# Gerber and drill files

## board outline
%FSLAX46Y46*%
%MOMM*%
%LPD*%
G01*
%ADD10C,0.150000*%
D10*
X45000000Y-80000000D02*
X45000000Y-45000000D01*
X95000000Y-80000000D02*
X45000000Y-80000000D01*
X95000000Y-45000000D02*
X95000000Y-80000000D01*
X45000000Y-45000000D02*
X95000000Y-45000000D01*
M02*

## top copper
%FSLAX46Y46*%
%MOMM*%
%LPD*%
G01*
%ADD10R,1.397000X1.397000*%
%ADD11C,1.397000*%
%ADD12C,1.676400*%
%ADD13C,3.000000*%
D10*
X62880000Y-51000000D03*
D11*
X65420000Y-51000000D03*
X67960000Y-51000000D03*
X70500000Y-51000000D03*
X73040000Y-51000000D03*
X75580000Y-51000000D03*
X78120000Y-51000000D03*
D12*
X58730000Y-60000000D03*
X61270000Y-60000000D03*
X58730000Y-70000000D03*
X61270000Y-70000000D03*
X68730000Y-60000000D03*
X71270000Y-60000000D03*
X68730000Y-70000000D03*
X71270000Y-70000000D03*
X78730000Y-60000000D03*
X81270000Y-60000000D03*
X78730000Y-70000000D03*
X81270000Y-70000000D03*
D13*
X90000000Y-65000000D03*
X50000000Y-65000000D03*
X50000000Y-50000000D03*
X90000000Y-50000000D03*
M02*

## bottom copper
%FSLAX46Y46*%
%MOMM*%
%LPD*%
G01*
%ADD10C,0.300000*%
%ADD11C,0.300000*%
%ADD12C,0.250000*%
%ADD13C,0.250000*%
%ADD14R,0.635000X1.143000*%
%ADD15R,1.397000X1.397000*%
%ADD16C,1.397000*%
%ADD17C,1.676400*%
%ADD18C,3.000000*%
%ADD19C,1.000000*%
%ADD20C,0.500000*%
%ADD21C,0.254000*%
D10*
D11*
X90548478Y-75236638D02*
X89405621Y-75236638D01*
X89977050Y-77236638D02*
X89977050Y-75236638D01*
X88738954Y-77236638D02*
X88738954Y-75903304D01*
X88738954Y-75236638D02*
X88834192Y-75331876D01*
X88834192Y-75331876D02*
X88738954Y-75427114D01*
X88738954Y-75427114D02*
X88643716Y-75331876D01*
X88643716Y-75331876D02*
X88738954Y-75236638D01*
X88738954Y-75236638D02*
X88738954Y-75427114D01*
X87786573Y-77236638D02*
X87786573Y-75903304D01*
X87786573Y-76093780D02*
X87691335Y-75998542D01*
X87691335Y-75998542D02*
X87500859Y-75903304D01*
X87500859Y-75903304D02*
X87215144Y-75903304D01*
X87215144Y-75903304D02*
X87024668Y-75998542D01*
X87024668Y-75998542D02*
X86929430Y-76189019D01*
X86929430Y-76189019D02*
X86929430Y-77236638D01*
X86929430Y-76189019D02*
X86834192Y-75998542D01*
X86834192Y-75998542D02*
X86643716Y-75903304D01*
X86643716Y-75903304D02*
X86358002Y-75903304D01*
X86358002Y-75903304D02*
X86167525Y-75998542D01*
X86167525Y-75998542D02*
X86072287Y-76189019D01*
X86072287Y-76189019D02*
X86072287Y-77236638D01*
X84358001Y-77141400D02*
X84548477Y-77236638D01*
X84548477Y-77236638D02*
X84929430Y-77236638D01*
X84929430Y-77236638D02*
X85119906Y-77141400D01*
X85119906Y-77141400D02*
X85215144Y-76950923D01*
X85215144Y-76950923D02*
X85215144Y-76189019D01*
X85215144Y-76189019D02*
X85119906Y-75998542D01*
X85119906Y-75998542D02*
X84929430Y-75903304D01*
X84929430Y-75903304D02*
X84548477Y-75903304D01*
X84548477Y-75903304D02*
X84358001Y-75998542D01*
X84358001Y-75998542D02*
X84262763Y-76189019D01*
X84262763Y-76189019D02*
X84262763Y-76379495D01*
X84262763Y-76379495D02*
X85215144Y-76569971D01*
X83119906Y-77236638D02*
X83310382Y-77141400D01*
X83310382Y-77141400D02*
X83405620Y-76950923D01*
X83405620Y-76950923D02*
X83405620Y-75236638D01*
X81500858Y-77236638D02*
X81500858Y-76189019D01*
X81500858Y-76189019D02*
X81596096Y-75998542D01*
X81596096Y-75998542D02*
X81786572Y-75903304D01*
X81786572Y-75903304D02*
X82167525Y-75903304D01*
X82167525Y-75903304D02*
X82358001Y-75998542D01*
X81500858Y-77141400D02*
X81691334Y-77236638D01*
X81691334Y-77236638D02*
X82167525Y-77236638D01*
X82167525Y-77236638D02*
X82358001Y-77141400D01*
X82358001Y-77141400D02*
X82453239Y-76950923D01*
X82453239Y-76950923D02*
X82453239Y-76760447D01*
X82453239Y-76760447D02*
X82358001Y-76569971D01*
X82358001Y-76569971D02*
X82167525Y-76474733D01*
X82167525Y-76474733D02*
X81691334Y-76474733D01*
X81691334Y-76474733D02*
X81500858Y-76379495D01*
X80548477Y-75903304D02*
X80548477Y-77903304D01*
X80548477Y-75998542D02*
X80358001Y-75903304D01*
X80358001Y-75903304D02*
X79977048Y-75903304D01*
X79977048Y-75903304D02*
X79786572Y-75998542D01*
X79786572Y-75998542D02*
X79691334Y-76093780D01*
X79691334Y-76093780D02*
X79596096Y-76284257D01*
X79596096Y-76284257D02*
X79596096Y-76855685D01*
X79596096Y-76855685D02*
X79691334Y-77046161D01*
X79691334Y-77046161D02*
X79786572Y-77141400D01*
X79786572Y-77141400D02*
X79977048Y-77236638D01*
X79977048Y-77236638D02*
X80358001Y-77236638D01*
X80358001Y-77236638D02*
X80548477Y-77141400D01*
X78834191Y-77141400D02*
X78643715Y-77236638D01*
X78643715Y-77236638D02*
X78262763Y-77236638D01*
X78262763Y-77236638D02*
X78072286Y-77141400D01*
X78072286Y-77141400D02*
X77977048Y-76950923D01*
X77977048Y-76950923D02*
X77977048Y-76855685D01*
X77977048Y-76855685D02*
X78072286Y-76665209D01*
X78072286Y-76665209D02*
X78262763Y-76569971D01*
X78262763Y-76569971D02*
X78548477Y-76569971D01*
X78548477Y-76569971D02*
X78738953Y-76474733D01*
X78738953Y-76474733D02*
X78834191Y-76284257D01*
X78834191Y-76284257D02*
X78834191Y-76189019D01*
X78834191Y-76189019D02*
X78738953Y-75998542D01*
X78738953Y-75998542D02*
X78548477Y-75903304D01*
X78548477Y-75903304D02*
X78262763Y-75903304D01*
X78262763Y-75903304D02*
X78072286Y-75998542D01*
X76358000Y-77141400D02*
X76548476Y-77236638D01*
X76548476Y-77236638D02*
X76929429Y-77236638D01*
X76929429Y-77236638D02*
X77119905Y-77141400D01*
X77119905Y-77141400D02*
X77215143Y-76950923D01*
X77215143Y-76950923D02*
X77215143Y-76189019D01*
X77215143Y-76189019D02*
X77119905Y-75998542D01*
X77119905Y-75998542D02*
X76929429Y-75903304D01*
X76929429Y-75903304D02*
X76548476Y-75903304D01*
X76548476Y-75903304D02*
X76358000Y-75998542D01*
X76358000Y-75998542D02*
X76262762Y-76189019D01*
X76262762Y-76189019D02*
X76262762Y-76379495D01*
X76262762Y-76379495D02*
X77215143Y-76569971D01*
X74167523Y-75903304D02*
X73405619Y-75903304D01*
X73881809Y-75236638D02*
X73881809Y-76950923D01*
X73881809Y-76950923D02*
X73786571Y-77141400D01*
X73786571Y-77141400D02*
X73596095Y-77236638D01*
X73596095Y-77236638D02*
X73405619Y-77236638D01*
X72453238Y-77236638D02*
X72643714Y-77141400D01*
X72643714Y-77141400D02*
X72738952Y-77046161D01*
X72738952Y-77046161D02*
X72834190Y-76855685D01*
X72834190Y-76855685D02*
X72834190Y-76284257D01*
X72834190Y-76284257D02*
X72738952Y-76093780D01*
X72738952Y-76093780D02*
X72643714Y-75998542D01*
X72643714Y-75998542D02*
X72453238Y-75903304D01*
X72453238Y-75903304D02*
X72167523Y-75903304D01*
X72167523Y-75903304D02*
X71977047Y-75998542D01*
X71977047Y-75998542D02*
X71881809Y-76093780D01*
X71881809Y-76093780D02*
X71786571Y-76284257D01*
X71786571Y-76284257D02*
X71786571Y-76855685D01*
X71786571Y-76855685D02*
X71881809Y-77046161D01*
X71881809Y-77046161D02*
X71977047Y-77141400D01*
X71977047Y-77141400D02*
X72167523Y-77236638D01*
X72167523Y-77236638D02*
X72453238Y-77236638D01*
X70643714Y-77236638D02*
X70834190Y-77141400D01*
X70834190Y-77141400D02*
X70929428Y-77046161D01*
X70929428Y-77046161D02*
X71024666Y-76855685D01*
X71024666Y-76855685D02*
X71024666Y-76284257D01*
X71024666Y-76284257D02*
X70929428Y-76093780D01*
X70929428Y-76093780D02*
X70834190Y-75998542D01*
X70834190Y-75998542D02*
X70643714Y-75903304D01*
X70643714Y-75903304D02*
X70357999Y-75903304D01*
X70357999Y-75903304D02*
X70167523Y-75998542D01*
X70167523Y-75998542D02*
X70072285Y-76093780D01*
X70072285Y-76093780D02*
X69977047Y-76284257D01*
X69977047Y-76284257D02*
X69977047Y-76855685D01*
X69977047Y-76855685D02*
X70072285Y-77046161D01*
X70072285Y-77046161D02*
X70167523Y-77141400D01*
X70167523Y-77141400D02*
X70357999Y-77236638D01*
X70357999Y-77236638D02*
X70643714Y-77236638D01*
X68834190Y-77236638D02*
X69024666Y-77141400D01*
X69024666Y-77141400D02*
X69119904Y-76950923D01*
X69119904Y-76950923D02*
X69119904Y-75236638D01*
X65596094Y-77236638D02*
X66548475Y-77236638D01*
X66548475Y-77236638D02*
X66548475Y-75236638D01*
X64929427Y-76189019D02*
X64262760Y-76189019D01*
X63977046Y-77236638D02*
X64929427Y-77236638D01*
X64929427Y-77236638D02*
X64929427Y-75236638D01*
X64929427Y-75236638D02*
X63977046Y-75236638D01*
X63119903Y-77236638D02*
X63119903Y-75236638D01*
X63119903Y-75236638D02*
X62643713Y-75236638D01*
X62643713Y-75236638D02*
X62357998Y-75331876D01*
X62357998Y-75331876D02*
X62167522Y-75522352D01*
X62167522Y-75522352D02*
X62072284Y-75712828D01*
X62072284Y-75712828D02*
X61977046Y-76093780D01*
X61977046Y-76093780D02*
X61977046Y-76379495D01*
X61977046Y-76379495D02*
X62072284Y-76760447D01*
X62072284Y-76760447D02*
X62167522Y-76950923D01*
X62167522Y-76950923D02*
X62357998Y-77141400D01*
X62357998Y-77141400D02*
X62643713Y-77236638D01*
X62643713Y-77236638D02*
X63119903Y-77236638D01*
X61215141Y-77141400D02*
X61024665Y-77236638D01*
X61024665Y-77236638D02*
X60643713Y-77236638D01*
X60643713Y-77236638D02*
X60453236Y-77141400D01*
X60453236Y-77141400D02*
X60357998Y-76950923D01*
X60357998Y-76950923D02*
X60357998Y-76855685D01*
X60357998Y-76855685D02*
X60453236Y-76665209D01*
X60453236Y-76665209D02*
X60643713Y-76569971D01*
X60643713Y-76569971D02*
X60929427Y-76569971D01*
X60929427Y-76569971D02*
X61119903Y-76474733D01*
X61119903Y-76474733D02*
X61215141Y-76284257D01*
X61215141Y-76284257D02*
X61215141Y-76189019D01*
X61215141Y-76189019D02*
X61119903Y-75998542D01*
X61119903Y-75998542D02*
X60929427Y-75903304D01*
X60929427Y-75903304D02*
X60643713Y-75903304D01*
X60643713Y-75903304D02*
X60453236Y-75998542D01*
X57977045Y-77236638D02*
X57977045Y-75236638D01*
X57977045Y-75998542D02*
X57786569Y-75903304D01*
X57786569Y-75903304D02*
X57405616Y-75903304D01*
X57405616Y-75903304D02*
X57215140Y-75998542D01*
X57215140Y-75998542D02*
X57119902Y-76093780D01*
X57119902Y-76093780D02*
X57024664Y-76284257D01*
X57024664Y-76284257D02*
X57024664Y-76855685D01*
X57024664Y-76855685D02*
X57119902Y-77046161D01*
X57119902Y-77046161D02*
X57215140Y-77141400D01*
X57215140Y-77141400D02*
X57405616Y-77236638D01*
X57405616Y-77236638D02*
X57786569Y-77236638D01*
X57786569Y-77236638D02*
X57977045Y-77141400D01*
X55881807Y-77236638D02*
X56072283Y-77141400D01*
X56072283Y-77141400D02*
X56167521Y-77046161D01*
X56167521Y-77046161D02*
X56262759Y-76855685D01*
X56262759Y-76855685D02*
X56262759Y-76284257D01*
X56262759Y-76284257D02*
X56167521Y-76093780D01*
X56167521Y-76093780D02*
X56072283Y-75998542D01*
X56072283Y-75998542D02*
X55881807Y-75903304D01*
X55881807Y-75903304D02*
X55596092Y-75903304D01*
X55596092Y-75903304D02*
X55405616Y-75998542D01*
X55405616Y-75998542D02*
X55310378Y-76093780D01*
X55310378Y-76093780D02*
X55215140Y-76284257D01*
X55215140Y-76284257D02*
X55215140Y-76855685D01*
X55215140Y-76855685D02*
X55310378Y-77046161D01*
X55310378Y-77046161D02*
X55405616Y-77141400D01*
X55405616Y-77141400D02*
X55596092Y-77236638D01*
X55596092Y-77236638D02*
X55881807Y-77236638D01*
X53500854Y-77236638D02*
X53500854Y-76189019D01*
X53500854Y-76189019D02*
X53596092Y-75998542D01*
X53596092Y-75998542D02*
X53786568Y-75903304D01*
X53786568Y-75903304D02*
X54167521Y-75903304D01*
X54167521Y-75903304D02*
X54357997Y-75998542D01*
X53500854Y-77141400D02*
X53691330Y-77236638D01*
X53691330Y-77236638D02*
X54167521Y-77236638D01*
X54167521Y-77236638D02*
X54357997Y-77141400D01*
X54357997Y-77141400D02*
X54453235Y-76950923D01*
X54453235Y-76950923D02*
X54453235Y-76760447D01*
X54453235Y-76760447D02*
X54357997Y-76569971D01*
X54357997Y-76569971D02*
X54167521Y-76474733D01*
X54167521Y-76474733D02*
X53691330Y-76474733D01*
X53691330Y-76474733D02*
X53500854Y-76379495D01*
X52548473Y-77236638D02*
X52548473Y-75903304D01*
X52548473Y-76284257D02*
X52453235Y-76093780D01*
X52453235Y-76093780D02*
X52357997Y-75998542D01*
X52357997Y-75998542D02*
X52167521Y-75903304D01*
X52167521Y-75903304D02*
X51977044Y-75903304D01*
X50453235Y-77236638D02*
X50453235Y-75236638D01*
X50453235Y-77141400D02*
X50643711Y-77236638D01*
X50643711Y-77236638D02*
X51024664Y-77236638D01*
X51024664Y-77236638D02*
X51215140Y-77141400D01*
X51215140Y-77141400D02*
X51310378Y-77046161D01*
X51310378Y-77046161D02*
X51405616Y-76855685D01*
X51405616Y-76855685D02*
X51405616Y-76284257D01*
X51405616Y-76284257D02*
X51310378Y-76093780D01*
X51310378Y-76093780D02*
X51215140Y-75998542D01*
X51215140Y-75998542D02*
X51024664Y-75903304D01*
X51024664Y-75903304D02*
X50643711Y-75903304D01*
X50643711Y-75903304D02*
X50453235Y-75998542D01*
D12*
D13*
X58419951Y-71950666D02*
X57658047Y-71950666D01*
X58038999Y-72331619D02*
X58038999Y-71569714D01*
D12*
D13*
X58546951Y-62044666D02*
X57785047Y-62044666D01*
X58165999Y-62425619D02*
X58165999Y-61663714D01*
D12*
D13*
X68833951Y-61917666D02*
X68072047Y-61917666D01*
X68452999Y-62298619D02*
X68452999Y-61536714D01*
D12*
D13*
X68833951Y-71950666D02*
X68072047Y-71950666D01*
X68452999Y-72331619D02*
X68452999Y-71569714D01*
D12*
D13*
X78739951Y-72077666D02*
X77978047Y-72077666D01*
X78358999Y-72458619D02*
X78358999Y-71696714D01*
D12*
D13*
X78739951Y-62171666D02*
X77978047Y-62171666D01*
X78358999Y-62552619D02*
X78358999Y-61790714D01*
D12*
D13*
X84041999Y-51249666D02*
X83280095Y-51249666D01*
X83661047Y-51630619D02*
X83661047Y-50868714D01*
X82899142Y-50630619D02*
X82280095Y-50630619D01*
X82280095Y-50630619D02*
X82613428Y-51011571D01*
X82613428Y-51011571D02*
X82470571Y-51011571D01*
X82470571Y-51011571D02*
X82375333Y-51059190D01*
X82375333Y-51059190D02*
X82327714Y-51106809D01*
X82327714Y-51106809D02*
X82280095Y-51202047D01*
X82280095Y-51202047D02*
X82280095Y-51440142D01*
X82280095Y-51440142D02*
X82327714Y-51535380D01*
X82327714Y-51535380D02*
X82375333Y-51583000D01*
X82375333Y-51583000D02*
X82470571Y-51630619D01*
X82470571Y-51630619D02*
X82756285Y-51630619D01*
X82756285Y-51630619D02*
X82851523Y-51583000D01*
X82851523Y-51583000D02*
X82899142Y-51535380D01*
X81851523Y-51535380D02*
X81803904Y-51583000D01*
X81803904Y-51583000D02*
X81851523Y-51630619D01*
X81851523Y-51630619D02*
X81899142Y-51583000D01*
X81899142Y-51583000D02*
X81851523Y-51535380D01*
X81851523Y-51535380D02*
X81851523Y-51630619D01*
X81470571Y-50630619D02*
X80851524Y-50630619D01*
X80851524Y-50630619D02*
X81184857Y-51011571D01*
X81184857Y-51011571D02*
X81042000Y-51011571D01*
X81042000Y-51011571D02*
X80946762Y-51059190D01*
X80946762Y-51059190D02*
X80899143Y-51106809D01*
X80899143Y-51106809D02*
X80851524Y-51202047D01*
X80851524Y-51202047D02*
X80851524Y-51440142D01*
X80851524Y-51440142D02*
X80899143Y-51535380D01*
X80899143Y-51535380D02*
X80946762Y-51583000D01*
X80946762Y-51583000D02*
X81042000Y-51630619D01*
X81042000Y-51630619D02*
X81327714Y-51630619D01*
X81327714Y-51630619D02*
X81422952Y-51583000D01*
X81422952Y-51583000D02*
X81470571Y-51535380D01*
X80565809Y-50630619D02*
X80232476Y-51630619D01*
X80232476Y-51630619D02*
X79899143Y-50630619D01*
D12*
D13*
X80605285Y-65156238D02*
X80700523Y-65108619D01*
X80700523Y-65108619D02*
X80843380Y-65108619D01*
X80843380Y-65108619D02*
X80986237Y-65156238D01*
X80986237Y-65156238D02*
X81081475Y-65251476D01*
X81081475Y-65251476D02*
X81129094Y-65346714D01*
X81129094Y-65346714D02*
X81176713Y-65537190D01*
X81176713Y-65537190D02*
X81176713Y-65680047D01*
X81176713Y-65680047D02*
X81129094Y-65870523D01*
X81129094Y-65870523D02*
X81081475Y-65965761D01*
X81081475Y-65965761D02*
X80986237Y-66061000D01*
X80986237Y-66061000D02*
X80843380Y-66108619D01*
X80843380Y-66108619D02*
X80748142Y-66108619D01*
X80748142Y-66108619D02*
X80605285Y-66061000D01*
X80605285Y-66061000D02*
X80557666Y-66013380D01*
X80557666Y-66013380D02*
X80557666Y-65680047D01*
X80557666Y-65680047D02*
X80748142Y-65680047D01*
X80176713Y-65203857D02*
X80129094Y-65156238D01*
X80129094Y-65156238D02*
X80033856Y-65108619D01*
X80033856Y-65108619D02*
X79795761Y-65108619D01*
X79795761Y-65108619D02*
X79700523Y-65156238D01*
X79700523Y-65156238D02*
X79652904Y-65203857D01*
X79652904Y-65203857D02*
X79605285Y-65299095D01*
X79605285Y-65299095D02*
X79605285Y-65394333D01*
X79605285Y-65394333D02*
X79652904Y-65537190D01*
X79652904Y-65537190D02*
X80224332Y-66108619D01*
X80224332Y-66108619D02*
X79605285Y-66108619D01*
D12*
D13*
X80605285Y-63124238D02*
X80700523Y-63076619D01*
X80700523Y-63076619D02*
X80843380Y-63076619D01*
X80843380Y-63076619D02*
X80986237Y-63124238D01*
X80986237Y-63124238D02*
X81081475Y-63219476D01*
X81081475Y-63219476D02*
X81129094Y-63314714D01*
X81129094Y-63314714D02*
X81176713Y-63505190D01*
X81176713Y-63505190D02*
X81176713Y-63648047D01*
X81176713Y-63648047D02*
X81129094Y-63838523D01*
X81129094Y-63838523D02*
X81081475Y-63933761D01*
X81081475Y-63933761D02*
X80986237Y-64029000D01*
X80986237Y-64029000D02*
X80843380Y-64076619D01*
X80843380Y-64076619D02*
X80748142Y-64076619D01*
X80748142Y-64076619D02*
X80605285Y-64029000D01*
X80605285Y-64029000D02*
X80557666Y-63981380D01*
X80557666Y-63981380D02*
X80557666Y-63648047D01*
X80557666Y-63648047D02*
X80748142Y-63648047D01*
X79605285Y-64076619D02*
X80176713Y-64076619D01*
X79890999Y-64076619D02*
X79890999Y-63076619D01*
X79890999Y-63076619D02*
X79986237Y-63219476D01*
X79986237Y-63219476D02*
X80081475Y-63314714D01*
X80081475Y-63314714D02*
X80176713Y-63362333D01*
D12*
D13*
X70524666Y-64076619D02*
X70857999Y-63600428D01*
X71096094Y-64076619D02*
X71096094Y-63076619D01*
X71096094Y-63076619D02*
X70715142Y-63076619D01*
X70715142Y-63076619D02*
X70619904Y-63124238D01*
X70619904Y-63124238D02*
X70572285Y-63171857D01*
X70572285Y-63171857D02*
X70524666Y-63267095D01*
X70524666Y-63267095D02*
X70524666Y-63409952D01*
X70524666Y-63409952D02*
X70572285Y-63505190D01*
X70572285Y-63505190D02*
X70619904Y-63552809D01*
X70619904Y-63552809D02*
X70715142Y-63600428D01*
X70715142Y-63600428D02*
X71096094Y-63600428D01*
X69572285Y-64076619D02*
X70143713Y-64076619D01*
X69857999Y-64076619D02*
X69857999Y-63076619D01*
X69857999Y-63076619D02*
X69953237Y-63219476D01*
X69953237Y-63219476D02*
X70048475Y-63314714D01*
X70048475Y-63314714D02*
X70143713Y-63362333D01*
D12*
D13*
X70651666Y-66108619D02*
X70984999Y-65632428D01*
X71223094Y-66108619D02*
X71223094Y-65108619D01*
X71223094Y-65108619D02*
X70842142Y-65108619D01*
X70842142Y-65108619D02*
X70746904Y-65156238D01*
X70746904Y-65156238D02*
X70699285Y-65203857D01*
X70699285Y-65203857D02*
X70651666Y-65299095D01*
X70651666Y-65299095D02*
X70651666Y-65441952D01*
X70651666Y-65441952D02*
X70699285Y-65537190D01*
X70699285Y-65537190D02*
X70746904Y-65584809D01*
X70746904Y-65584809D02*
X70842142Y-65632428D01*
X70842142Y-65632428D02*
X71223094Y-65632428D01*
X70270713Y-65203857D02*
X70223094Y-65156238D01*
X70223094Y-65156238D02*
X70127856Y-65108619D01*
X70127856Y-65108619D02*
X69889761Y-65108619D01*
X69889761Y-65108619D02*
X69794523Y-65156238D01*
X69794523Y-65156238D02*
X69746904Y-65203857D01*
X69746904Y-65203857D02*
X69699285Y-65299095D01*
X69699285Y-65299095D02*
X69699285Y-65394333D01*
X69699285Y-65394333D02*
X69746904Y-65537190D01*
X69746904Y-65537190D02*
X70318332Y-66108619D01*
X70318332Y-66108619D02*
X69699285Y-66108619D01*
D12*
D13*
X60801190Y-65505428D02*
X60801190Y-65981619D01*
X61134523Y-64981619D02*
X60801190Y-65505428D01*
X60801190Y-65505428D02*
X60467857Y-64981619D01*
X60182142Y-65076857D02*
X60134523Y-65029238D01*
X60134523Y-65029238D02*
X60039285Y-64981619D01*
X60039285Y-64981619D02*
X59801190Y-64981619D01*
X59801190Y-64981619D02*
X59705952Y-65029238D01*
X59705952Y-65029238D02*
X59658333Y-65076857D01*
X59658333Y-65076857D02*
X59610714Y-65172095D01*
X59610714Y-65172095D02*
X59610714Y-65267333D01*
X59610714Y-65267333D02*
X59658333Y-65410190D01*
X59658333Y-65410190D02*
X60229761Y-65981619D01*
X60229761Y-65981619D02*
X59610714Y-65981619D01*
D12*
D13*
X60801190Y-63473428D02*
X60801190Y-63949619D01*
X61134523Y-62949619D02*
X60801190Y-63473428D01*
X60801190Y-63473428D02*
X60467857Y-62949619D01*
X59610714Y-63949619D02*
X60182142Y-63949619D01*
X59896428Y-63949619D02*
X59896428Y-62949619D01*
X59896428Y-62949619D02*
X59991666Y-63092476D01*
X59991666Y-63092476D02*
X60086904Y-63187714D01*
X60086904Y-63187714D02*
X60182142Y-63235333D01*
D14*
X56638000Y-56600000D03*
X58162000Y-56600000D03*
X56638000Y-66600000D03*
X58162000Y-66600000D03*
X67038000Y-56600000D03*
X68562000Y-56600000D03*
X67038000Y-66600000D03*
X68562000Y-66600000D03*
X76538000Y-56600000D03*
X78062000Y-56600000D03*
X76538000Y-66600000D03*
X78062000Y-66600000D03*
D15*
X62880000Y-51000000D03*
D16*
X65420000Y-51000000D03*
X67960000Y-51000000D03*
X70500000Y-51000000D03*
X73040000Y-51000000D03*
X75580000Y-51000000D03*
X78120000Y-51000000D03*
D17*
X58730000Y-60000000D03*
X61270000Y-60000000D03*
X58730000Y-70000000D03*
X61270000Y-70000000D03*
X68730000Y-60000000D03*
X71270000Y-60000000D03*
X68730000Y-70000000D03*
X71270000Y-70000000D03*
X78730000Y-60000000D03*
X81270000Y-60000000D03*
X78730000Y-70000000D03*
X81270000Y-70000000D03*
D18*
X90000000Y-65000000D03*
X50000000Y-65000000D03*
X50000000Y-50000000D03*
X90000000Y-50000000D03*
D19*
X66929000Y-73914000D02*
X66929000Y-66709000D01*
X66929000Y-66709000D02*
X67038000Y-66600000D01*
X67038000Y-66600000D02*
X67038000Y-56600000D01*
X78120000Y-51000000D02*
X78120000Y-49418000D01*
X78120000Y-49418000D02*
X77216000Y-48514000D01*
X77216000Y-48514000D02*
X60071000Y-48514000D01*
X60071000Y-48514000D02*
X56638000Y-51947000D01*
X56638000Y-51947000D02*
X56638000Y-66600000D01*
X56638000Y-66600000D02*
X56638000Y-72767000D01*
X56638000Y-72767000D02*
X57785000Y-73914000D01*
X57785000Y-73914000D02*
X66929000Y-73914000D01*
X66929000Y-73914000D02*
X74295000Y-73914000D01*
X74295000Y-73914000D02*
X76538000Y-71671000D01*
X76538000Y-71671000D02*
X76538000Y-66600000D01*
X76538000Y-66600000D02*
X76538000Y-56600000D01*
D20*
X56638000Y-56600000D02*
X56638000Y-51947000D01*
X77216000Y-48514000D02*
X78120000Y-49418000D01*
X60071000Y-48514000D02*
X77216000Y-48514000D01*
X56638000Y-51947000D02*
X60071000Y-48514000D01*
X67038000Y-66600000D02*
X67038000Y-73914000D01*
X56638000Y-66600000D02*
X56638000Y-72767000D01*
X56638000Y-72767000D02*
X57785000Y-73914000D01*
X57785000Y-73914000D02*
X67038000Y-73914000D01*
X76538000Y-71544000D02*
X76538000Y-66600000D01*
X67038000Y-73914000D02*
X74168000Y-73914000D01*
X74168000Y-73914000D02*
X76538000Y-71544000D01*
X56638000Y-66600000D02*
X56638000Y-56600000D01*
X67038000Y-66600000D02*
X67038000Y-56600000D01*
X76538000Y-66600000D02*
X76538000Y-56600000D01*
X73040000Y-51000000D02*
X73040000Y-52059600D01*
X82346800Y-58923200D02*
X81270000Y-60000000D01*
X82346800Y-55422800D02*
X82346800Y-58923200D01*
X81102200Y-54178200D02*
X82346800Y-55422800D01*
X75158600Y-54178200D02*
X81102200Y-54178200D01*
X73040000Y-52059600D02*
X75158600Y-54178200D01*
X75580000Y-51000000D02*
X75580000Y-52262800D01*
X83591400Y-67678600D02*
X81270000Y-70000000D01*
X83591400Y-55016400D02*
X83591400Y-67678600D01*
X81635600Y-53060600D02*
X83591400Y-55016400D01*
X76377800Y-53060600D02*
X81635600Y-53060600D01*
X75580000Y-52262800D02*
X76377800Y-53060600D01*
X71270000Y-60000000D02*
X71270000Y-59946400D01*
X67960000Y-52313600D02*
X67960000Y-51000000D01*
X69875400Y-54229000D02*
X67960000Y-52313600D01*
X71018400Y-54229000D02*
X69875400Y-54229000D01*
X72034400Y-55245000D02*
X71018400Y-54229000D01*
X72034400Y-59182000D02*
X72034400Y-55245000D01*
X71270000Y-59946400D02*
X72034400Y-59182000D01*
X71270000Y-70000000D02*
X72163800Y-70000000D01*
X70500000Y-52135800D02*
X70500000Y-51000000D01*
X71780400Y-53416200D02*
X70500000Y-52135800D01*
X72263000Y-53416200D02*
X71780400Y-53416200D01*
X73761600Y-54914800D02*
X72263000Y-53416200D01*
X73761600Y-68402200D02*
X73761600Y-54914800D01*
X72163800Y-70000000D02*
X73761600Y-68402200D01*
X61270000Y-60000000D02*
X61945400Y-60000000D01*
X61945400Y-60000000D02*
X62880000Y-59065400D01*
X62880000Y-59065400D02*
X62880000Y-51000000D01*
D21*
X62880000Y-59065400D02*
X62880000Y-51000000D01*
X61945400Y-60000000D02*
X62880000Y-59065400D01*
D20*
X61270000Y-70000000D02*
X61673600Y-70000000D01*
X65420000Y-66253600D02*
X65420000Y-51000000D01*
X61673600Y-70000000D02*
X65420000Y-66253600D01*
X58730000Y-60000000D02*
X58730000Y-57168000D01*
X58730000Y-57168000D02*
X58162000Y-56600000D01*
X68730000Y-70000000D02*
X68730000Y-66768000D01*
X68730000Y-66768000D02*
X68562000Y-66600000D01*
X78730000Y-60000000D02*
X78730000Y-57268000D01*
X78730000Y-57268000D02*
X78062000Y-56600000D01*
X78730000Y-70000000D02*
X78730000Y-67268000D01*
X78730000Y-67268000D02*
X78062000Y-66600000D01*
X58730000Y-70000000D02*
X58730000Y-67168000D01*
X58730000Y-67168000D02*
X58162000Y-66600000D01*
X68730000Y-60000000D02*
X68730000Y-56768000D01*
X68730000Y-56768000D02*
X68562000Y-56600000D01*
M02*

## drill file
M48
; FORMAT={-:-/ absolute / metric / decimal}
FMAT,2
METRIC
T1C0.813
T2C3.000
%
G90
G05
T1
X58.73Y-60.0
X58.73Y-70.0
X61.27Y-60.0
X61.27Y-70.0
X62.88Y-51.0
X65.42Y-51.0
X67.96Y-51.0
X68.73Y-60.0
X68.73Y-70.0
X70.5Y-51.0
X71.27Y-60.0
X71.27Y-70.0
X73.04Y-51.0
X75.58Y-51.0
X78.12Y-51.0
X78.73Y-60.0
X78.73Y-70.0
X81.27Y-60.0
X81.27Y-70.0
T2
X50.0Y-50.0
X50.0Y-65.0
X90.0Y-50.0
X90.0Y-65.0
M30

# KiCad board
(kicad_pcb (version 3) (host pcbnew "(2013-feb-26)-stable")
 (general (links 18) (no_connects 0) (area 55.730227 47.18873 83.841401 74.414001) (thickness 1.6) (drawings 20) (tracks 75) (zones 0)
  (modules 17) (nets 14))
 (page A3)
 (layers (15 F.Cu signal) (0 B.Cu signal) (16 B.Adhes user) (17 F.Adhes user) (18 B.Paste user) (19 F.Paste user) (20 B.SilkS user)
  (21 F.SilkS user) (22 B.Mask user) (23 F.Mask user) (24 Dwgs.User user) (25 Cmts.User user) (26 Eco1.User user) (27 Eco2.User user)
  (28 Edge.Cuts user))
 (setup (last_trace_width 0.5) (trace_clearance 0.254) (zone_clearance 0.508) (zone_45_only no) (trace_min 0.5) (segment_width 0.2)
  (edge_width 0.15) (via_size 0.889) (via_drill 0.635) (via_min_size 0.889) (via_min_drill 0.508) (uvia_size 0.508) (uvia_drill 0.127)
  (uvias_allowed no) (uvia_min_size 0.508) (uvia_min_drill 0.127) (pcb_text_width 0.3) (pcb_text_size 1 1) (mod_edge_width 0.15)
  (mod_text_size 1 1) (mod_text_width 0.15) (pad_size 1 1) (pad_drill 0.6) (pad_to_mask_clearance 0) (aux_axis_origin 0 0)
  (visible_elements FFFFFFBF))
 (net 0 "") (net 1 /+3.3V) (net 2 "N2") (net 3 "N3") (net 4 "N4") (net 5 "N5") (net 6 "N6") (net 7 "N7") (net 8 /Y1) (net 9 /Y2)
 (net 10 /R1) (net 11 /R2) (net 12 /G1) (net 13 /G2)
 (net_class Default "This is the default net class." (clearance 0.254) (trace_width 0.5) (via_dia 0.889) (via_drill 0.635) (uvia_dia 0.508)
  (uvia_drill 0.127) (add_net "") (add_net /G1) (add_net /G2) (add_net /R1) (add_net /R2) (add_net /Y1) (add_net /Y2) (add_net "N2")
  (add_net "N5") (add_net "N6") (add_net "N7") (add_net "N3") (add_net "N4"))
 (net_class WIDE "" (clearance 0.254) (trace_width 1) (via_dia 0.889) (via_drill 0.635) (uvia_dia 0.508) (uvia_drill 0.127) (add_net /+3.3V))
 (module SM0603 (layer B.Cu) (at 57.4 56.6)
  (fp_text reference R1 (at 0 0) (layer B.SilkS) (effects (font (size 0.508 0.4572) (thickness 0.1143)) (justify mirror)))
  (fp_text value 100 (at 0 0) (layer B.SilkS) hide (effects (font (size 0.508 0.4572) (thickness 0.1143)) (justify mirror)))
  (pad 1 smd rect (at -0.762 0) (size 0.635 1.143) (layers B.Cu B.Paste B.Mask) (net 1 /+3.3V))
  (pad 2 smd rect (at 0.762 0) (size 0.635 1.143) (layers B.Cu B.Paste B.Mask) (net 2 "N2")))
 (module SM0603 (layer B.Cu) (at 57.4 66.6)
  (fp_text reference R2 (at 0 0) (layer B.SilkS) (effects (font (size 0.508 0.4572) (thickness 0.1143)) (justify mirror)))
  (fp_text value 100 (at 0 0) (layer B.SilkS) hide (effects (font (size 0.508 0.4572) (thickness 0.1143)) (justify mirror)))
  (pad 1 smd rect (at -0.762 0) (size 0.635 1.143) (layers B.Cu B.Paste B.Mask) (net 1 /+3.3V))
  (pad 2 smd rect (at 0.762 0) (size 0.635 1.143) (layers B.Cu B.Paste B.Mask) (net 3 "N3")))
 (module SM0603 (layer B.Cu) (at 67.8 56.6)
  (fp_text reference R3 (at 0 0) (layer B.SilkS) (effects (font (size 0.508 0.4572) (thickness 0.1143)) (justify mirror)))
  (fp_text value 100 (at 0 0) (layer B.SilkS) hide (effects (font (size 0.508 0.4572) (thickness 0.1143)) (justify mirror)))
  (pad 1 smd rect (at -0.762 0) (size 0.635 1.143) (layers B.Cu B.Paste B.Mask) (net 1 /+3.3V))
  (pad 2 smd rect (at 0.762 0) (size 0.635 1.143) (layers B.Cu B.Paste B.Mask) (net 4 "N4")))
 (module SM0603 (layer B.Cu) (at 67.8 66.6)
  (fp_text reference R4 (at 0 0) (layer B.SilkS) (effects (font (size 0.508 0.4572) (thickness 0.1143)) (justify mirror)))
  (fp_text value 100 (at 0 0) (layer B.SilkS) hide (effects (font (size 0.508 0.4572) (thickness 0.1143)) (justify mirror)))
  (pad 1 smd rect (at -0.762 0) (size 0.635 1.143) (layers B.Cu B.Paste B.Mask) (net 1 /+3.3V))
  (pad 2 smd rect (at 0.762 0) (size 0.635 1.143) (layers B.Cu B.Paste B.Mask) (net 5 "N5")))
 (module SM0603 (layer B.Cu) (at 77.3 56.6)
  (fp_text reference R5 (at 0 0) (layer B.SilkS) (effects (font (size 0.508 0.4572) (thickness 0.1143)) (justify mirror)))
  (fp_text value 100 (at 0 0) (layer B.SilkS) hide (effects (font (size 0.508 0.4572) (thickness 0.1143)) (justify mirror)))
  (pad 1 smd rect (at -0.762 0) (size 0.635 1.143) (layers B.Cu B.Paste B.Mask) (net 1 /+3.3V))
  (pad 2 smd rect (at 0.762 0) (size 0.635 1.143) (layers B.Cu B.Paste B.Mask) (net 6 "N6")))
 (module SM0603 (layer B.Cu) (at 77.3 66.6)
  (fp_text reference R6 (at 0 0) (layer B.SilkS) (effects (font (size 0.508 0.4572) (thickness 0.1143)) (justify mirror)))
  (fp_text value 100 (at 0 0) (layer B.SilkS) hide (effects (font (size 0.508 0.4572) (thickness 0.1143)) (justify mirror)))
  (pad 1 smd rect (at -0.762 0) (size 0.635 1.143) (layers B.Cu B.Paste B.Mask) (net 1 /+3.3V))
  (pad 2 smd rect (at 0.762 0) (size 0.635 1.143) (layers B.Cu B.Paste B.Mask) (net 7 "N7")))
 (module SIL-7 (layer F.Cu) (at 70.5 51)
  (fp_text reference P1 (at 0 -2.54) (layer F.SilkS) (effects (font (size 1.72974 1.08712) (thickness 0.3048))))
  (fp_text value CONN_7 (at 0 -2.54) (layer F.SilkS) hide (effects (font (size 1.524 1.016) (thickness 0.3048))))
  (pad 1 thru_hole rect (at -7.62 0) (size 1.397 1.397) (drill 0.8128) (layers *.Cu *.Mask F.SilkS) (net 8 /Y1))
  (pad 2 thru_hole circle (at -5.08 0) (size 1.397 1.397) (drill 0.8128) (layers *.Cu *.SilkS *.Mask) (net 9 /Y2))
  (pad 3 thru_hole circle (at -2.54 0) (size 1.397 1.397) (drill 0.8128) (layers *.Cu *.SilkS *.Mask) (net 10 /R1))
  (pad 4 thru_hole circle (at 0 0) (size 1.397 1.397) (drill 0.8128) (layers *.Cu *.SilkS *.Mask) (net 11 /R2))
  (pad 5 thru_hole circle (at 2.54 0) (size 1.397 1.397) (drill 0.8128) (layers *.Cu *.SilkS *.Mask) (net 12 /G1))
  (pad 6 thru_hole circle (at 5.08 0) (size 1.397 1.397) (drill 0.8128) (layers *.Cu *.SilkS *.Mask) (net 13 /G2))
  (pad 7 thru_hole circle (at 7.62 0) (size 1.397 1.397) (drill 0.8128) (layers *.Cu *.SilkS *.Mask) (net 1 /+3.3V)))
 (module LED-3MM (layer F.Cu) (at 60 60)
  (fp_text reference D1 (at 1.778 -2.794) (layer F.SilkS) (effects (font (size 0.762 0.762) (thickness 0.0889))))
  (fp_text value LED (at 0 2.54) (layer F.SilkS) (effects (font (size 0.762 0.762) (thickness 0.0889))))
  (pad 1 thru_hole circle (at -1.27 0) (size 1.6764 1.6764) (drill 0.8128) (layers *.Cu F.Paste F.SilkS F.Mask) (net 2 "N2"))
  (pad 2 thru_hole circle (at 1.27 0) (size 1.6764 1.6764) (drill 0.8128) (layers *.Cu F.Paste F.SilkS F.Mask) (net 8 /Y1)))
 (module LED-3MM (layer F.Cu) (at 60 70)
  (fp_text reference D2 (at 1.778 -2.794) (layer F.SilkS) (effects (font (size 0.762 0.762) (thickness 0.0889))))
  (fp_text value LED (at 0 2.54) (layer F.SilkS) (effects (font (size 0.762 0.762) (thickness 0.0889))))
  (pad 1 thru_hole circle (at -1.27 0) (size 1.6764 1.6764) (drill 0.8128) (layers *.Cu F.Paste F.SilkS F.Mask) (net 3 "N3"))
  (pad 2 thru_hole circle (at 1.27 0) (size 1.6764 1.6764) (drill 0.8128) (layers *.Cu F.Paste F.SilkS F.Mask) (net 9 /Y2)))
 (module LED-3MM (layer F.Cu) (at 70 60)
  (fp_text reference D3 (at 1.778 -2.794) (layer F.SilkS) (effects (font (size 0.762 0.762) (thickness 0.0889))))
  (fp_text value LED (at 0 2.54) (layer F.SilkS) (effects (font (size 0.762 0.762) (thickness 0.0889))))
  (pad 1 thru_hole circle (at -1.27 0) (size 1.6764 1.6764) (drill 0.8128) (layers *.Cu F.Paste F.SilkS F.Mask) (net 4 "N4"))
  (pad 2 thru_hole circle (at 1.27 0) (size 1.6764 1.6764) (drill 0.8128) (layers *.Cu F.Paste F.SilkS F.Mask) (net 10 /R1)))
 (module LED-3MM (layer F.Cu) (at 70 70)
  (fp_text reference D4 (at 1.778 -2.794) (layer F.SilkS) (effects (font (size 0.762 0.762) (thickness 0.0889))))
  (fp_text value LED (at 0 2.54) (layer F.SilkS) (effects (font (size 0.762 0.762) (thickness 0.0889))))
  (pad 1 thru_hole circle (at -1.27 0) (size 1.6764 1.6764) (drill 0.8128) (layers *.Cu F.Paste F.SilkS F.Mask) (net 5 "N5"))
  (pad 2 thru_hole circle (at 1.27 0) (size 1.6764 1.6764) (drill 0.8128) (layers *.Cu F.Paste F.SilkS F.Mask) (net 11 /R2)))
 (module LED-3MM (layer F.Cu) (at 80 60)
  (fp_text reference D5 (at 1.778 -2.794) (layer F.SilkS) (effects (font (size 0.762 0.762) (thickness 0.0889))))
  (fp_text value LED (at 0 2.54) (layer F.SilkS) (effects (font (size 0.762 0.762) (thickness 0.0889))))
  (pad 1 thru_hole circle (at -1.27 0) (size 1.6764 1.6764) (drill 0.8128) (layers *.Cu F.Paste F.SilkS F.Mask) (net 6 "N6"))
  (pad 2 thru_hole circle (at 1.27 0) (size 1.6764 1.6764) (drill 0.8128) (layers *.Cu F.Paste F.SilkS F.Mask) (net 12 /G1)))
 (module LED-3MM (layer F.Cu) (at 80 70)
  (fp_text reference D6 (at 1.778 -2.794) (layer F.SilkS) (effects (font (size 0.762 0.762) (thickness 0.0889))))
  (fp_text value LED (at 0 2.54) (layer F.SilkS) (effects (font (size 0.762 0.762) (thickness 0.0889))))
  (pad 1 thru_hole circle (at -1.27 0) (size 1.6764 1.6764) (drill 0.8128) (layers *.Cu F.Paste F.SilkS F.Mask) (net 7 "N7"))
  (pad 2 thru_hole circle (at 1.27 0) (size 1.6764 1.6764) (drill 0.8128) (layers *.Cu F.Paste F.SilkS F.Mask) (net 13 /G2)))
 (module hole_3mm (layer F.Cu) (at 90 65)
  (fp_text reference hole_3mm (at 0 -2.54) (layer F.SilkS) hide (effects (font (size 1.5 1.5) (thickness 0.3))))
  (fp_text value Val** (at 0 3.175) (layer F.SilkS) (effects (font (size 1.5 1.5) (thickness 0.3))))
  (pad "" thru_hole circle (at 0 0) (size 3 3) (drill 3) (layers *.Cu F.SilkS)))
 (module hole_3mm (layer F.Cu) (at 50 65)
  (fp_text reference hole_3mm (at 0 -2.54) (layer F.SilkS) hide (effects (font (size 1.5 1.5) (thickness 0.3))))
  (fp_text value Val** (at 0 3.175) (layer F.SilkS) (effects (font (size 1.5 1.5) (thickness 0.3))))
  (pad "" thru_hole circle (at 0 0) (size 3 3) (drill 3) (layers *.Cu F.SilkS)))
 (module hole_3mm (layer F.Cu) (at 50 50)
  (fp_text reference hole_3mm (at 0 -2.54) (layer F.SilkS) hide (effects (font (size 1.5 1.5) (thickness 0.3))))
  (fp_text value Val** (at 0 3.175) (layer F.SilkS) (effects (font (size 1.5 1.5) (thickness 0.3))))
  (pad "" thru_hole circle (at 0 0) (size 3 3) (drill 3) (layers *.Cu F.SilkS)))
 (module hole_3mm (layer F.Cu) (at 90 50)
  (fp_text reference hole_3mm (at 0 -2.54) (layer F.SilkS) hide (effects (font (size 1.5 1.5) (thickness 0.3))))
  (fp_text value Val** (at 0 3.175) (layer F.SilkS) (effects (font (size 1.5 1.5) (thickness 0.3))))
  (pad "" thru_hole circle (at 0 0) (size 3 3) (drill 3) (layers *.Cu F.SilkS)))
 (gr_line (start 45 80) (end 45 45) (angle 90) (layer Edge.Cuts) (width 0.15))
 (gr_line (start 95 80) (end 45 80) (angle 90) (layer Edge.Cuts) (width 0.15))
 (gr_line (start 95 45) (end 95 80) (angle 90) (layer Edge.Cuts) (width 0.15))
 (gr_line (start 45 45) (end 95 45) (angle 90) (layer Edge.Cuts) (width 0.15))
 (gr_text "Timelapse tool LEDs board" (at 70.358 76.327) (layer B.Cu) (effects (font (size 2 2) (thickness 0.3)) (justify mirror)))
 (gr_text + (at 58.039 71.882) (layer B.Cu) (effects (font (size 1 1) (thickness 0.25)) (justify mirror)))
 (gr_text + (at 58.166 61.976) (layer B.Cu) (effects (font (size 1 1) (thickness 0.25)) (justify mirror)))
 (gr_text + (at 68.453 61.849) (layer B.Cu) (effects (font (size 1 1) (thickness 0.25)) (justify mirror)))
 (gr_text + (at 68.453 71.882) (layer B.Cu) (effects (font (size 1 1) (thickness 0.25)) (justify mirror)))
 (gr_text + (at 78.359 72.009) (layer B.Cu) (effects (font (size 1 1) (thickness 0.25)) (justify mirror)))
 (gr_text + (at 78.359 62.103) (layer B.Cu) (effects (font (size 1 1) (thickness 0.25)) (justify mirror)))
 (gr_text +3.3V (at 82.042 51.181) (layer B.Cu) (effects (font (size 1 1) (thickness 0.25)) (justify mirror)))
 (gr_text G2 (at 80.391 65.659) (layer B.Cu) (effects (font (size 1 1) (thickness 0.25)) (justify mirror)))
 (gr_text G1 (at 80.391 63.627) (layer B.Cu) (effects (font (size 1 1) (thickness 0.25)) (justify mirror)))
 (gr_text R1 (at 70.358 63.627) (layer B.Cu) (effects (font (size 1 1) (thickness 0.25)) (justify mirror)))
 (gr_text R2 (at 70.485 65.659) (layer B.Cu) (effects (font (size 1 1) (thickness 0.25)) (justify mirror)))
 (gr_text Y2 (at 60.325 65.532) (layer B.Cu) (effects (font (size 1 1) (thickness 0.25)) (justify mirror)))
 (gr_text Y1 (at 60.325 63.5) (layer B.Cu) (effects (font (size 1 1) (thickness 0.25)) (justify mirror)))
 (segment (start 66.929 73.914) (end 66.929 66.709) (width 1) (layer B.Cu) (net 1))
 (segment (start 66.929 66.709) (end 67.038 66.6) (width 1) (layer B.Cu) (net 1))
 (segment (start 67.038 66.6) (end 67.038 56.6) (width 1) (layer B.Cu) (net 1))
 (segment (start 78.12 51) (end 78.12 49.418) (width 1) (layer B.Cu) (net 1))
 (segment (start 78.12 49.418) (end 77.216 48.514) (width 1) (layer B.Cu) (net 1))
 (segment (start 77.216 48.514) (end 60.071 48.514) (width 1) (layer B.Cu) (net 1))
 (segment (start 60.071 48.514) (end 56.638 51.947) (width 1) (layer B.Cu) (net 1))
 (segment (start 56.638 51.947) (end 56.638 66.6) (width 1) (layer B.Cu) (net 1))
 (segment (start 56.638 66.6) (end 56.638 72.767) (width 1) (layer B.Cu) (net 1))
 (segment (start 56.638 72.767) (end 57.785 73.914) (width 1) (layer B.Cu) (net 1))
 (segment (start 57.785 73.914) (end 66.929 73.914) (width 1) (layer B.Cu) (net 1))
 (segment (start 66.929 73.914) (end 74.295 73.914) (width 1) (layer B.Cu) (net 1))
 (segment (start 74.295 73.914) (end 76.538 71.671) (width 1) (layer B.Cu) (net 1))
 (segment (start 76.538 71.671) (end 76.538 66.6) (width 1) (layer B.Cu) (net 1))
 (segment (start 76.538 66.6) (end 76.538 56.6) (width 1) (layer B.Cu) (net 1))
 (segment (start 56.638 56.6) (end 56.638 51.947) (width 0.5) (layer B.Cu) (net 1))
 (segment (start 77.216 48.514) (end 78.12 49.418) (width 0.5) (layer B.Cu) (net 1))
 (segment (start 60.071 48.514) (end 77.216 48.514) (width 0.5) (layer B.Cu) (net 1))
 (segment (start 56.638 51.947) (end 60.071 48.514) (width 0.5) (layer B.Cu) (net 1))
 (segment (start 67.038 66.6) (end 67.038 73.914) (width 0.5) (layer B.Cu) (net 1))
 (segment (start 56.638 66.6) (end 56.638 72.767) (width 0.5) (layer B.Cu) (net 1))
 (segment (start 56.638 72.767) (end 57.785 73.914) (width 0.5) (layer B.Cu) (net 1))
 (segment (start 57.785 73.914) (end 67.038 73.914) (width 0.5) (layer B.Cu) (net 1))
 (segment (start 76.538 71.544) (end 76.538 66.6) (width 0.5) (layer B.Cu) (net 1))
 (segment (start 67.038 73.914) (end 74.168 73.914) (width 0.5) (layer B.Cu) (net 1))
 (segment (start 74.168 73.914) (end 76.538 71.544) (width 0.5) (layer B.Cu) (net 1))
 (segment (start 56.638 66.6) (end 56.638 56.6) (width 0.5) (layer B.Cu) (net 1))
 (segment (start 67.038 66.6) (end 67.038 56.6) (width 0.5) (layer B.Cu) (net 1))
 (segment (start 76.538 66.6) (end 76.538 56.6) (width 0.5) (layer B.Cu) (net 1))
 (segment (start 73.04 51) (end 73.04 52.0596) (width 0.5) (layer B.Cu) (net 12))
 (segment (start 82.3468 58.9232) (end 81.27 60) (width 0.5) (layer B.Cu) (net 12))
 (segment (start 82.3468 55.4228) (end 82.3468 58.9232) (width 0.5) (layer B.Cu) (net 12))
 (segment (start 81.1022 54.1782) (end 82.3468 55.4228) (width 0.5) (layer B.Cu) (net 12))
 (segment (start 75.1586 54.1782) (end 81.1022 54.1782) (width 0.5) (layer B.Cu) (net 12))
 (segment (start 73.04 52.0596) (end 75.1586 54.1782) (width 0.5) (layer B.Cu) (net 12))
 (segment (start 75.58 51) (end 75.58 52.2628) (width 0.5) (layer B.Cu) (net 13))
 (segment (start 83.5914 67.6786) (end 81.27 70) (width 0.5) (layer B.Cu) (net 13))
 (segment (start 83.5914 55.0164) (end 83.5914 67.6786) (width 0.5) (layer B.Cu) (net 13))
 (segment (start 81.6356 53.0606) (end 83.5914 55.0164) (width 0.5) (layer B.Cu) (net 13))
 (segment (start 76.3778 53.0606) (end 81.6356 53.0606) (width 0.5) (layer B.Cu) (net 13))
 (segment (start 75.58 52.2628) (end 76.3778 53.0606) (width 0.5) (layer B.Cu) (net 13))
 (segment (start 71.27 60) (end 71.27 59.9464) (width 0.5) (layer B.Cu) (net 10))
 (segment (start 67.96 52.3136) (end 67.96 51) (width 0.5) (layer B.Cu) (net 10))
 (segment (start 69.8754 54.229) (end 67.96 52.3136) (width 0.5) (layer B.Cu) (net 10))
 (segment (start 71.0184 54.229) (end 69.8754 54.229) (width 0.5) (layer B.Cu) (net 10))
 (segment (start 72.0344 55.245) (end 71.0184 54.229) (width 0.5) (layer B.Cu) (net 10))
 (segment (start 72.0344 59.182) (end 72.0344 55.245) (width 0.5) (layer B.Cu) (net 10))
 (segment (start 71.27 59.9464) (end 72.0344 59.182) (width 0.5) (layer B.Cu) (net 10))
 (segment (start 71.27 70) (end 72.1638 70) (width 0.5) (layer B.Cu) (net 11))
 (segment (start 70.5 52.1358) (end 70.5 51) (width 0.5) (layer B.Cu) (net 11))
 (segment (start 71.7804 53.4162) (end 70.5 52.1358) (width 0.5) (layer B.Cu) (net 11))
 (segment (start 72.263 53.4162) (end 71.7804 53.4162) (width 0.5) (layer B.Cu) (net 11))
 (segment (start 73.7616 54.9148) (end 72.263 53.4162) (width 0.5) (layer B.Cu) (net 11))
 (segment (start 73.7616 68.4022) (end 73.7616 54.9148) (width 0.5) (layer B.Cu) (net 11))
 (segment (start 72.1638 70) (end 73.7616 68.4022) (width 0.5) (layer B.Cu) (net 11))
 (segment (start 61.27 60) (end 61.9454 60) (width 0.5) (layer B.Cu) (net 8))
 (segment (start 61.9454 60) (end 62.88 59.0654) (width 0.5) (layer B.Cu) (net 8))
 (segment (start 62.88 59.0654) (end 62.88 51) (width 0.5) (layer B.Cu) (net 8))
 (segment (start 62.88 59.0654) (end 62.88 51) (width 0.254) (layer B.Cu) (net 8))
 (segment (start 61.9454 60) (end 62.88 59.0654) (width 0.254) (layer B.Cu) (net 8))
 (segment (start 61.27 70) (end 61.6736 70) (width 0.5) (layer B.Cu) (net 9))
 (segment (start 65.42 66.2536) (end 65.42 51) (width 0.5) (layer B.Cu) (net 9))
 (segment (start 61.6736 70) (end 65.42 66.2536) (width 0.5) (layer B.Cu) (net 9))
 (segment (start 58.73 60) (end 58.73 57.168) (width 0.5) (layer B.Cu) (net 2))
 (segment (start 58.73 57.168) (end 58.162 56.6) (width 0.5) (layer B.Cu) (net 2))
 (segment (start 68.73 70) (end 68.73 66.768) (width 0.5) (layer B.Cu) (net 5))
 (segment (start 68.73 66.768) (end 68.562 66.6) (width 0.5) (layer B.Cu) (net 5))
 (segment (start 78.73 60) (end 78.73 57.268) (width 0.5) (layer B.Cu) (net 6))
 (segment (start 78.73 57.268) (end 78.062 56.6) (width 0.5) (layer B.Cu) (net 6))
 (segment (start 78.73 70) (end 78.73 67.268) (width 0.5) (layer B.Cu) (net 7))
 (segment (start 78.73 67.268) (end 78.062 66.6) (width 0.5) (layer B.Cu) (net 7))
 (segment (start 58.73 70) (end 58.73 67.168) (width 0.5) (layer B.Cu) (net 3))
 (segment (start 58.73 67.168) (end 58.162 66.6) (width 0.5) (layer B.Cu) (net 3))
 (segment (start 68.73 60) (end 68.73 56.768) (width 0.5) (layer B.Cu) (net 4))
 (segment (start 68.73 56.768) (end 68.562 56.6) (width 0.5) (layer B.Cu) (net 4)))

